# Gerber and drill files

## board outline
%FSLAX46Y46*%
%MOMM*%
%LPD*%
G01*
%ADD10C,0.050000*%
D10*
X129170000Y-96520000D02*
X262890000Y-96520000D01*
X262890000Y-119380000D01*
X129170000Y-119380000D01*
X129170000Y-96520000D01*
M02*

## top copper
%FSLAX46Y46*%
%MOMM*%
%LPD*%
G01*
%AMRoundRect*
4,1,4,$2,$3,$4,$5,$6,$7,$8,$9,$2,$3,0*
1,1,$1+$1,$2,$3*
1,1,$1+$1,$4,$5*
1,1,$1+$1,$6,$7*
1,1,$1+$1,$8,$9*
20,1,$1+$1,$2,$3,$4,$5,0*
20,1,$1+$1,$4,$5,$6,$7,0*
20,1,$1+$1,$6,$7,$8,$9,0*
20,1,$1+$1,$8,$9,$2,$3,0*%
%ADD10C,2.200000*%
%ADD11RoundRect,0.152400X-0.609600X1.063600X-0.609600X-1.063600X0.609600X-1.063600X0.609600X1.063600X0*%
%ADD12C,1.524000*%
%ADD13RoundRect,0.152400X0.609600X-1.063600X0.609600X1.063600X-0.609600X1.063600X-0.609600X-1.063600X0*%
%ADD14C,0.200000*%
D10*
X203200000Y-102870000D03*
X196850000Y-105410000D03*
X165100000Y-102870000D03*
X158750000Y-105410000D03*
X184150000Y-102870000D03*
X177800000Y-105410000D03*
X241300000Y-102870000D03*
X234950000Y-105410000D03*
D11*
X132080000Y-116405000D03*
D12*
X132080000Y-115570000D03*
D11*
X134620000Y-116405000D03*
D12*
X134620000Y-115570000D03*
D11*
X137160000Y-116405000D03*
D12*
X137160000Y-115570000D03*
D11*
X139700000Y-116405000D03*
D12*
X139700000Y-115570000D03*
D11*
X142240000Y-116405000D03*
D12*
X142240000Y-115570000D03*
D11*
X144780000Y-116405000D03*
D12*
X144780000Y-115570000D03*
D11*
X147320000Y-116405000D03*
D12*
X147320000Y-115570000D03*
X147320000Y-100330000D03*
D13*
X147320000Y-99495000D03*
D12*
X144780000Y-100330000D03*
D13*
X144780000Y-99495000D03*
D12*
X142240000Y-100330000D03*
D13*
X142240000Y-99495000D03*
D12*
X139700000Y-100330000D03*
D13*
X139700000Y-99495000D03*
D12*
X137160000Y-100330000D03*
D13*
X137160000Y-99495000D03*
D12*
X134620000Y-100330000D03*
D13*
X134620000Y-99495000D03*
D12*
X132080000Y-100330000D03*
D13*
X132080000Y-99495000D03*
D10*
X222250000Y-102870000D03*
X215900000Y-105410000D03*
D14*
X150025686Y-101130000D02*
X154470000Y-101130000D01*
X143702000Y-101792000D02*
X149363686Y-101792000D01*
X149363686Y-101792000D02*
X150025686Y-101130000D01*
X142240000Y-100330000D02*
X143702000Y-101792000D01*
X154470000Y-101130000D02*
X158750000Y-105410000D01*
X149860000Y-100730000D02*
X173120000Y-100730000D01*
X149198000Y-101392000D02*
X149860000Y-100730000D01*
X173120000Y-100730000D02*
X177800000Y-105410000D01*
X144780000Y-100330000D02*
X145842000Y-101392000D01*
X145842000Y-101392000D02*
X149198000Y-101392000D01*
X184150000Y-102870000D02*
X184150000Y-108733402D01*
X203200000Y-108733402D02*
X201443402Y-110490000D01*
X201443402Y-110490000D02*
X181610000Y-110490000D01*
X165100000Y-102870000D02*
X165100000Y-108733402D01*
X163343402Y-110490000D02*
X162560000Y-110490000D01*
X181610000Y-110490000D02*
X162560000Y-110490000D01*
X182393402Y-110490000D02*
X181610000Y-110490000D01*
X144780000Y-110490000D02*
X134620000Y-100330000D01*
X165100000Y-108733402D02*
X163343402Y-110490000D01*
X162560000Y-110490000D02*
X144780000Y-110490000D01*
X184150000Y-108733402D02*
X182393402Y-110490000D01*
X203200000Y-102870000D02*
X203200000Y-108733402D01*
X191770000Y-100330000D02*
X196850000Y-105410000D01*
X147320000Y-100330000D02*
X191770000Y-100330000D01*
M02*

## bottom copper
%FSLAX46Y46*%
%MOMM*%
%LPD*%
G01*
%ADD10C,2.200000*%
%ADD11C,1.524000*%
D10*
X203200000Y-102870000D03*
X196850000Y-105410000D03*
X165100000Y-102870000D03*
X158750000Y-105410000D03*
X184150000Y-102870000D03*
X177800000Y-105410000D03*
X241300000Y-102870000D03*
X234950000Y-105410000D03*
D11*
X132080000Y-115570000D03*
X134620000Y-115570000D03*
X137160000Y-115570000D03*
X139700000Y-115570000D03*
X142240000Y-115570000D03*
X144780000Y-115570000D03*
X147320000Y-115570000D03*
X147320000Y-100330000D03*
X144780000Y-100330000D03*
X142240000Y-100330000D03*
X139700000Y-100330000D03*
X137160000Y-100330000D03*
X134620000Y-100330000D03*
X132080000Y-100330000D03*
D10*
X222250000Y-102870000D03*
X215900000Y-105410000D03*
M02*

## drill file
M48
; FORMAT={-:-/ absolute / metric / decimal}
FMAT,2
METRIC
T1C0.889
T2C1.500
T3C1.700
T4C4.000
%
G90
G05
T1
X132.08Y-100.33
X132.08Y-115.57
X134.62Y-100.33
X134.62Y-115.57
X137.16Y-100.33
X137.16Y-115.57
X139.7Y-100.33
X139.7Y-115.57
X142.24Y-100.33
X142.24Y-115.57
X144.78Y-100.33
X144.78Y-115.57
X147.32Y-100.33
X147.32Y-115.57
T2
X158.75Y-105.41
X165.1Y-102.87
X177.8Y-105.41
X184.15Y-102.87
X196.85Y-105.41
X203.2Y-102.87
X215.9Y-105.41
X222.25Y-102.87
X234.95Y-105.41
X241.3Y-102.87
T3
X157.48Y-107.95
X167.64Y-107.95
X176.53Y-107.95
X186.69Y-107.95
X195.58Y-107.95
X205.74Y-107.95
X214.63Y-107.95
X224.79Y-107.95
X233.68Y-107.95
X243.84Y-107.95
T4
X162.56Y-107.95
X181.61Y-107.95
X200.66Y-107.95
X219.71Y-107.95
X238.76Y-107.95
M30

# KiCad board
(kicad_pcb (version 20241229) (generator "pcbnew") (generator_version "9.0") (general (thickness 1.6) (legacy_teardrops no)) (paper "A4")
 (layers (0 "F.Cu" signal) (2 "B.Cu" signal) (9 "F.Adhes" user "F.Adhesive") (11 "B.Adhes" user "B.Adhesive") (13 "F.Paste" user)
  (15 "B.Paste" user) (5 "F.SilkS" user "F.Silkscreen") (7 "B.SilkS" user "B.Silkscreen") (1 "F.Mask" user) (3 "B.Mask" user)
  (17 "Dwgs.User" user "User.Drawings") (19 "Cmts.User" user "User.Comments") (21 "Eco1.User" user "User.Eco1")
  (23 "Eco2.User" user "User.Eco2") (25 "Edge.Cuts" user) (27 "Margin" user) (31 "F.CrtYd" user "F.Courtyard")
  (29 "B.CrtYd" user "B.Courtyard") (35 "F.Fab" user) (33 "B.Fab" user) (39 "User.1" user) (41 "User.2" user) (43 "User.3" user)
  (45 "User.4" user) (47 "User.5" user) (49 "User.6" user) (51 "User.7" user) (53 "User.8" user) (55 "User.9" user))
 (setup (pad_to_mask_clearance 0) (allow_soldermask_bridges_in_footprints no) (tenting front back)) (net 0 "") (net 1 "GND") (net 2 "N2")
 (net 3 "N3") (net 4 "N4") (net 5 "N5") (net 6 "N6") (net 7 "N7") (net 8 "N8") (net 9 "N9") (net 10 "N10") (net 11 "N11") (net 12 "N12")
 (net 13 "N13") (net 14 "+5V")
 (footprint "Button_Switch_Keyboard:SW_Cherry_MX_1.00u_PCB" (layer "F.Cu") (at 203.2 102.87)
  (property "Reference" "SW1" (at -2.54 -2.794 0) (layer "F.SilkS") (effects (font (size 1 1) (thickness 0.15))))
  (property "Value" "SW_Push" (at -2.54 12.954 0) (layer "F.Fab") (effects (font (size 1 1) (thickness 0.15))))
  (pad "" np_thru_hole circle (at -7.62 5.08) (size 1.7 1.7) (drill 1.7) (layers "*.Cu" "*.Mask"))
  (pad "" np_thru_hole circle (at -2.54 5.08) (size 4 4) (drill 4) (layers "*.Cu" "*.Mask"))
  (pad "" np_thru_hole circle (at 2.54 5.08) (size 1.7 1.7) (drill 1.7) (layers "*.Cu" "*.Mask"))
  (pad "1" thru_hole circle (at 0 0) (size 2.2 2.2) (drill 1.5) (layers "*.Cu" "*.Mask") (remove_unused_layers no) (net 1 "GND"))
  (pad "2" thru_hole circle (at -6.35 2.54) (size 2.2 2.2) (drill 1.5) (layers "*.Cu" "*.Mask") (remove_unused_layers no) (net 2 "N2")))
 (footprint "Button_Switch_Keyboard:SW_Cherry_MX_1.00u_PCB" (layer "F.Cu") (at 165.1 102.87)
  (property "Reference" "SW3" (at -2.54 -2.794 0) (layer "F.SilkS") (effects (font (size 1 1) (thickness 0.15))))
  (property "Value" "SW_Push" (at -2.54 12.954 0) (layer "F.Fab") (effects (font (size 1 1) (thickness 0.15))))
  (pad "" np_thru_hole circle (at -7.62 5.08) (size 1.7 1.7) (drill 1.7) (layers "*.Cu" "*.Mask"))
  (pad "" np_thru_hole circle (at -2.54 5.08) (size 4 4) (drill 4) (layers "*.Cu" "*.Mask"))
  (pad "" np_thru_hole circle (at 2.54 5.08) (size 1.7 1.7) (drill 1.7) (layers "*.Cu" "*.Mask"))
  (pad "1" thru_hole circle (at 0 0) (size 2.2 2.2) (drill 1.5) (layers "*.Cu" "*.Mask") (remove_unused_layers no) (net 1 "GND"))
  (pad "2" thru_hole circle (at -6.35 2.54) (size 2.2 2.2) (drill 1.5) (layers "*.Cu" "*.Mask") (remove_unused_layers no) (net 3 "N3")))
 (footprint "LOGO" (layer "F.Cu") (at 253.109093 100.484313)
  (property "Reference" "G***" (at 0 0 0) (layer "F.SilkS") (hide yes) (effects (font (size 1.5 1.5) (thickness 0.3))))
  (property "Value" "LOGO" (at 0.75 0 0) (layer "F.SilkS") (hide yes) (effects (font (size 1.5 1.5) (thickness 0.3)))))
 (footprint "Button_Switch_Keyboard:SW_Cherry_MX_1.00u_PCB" (layer "F.Cu") (at 184.15 102.87)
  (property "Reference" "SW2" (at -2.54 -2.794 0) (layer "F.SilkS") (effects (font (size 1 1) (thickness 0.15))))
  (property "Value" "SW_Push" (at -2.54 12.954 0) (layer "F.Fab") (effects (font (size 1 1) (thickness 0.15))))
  (pad "" np_thru_hole circle (at -7.62 5.08) (size 1.7 1.7) (drill 1.7) (layers "*.Cu" "*.Mask"))
  (pad "" np_thru_hole circle (at -2.54 5.08) (size 4 4) (drill 4) (layers "*.Cu" "*.Mask"))
  (pad "" np_thru_hole circle (at 2.54 5.08) (size 1.7 1.7) (drill 1.7) (layers "*.Cu" "*.Mask"))
  (pad "1" thru_hole circle (at 0 0) (size 2.2 2.2) (drill 1.5) (layers "*.Cu" "*.Mask") (remove_unused_layers no) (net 1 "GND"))
  (pad "2" thru_hole circle (at -6.35 2.54) (size 2.2 2.2) (drill 1.5) (layers "*.Cu" "*.Mask") (remove_unused_layers no) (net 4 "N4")))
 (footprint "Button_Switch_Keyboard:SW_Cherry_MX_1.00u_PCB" (layer "F.Cu") (at 241.3 102.87)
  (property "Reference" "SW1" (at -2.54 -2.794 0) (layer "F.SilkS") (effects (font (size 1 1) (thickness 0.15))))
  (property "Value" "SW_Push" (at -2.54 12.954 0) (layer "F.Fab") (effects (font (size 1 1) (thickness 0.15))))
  (pad "" np_thru_hole circle (at -7.62 5.08) (size 1.7 1.7) (drill 1.7) (layers "*.Cu" "*.Mask"))
  (pad "" np_thru_hole circle (at -2.54 5.08) (size 4 4) (drill 4) (layers "*.Cu" "*.Mask"))
  (pad "" np_thru_hole circle (at 2.54 5.08) (size 1.7 1.7) (drill 1.7) (layers "*.Cu" "*.Mask"))
  (pad "1" thru_hole circle (at 0 0) (size 2.2 2.2) (drill 1.5) (layers "*.Cu" "*.Mask") (remove_unused_layers no))
  (pad "2" thru_hole circle (at -6.35 2.54) (size 2.2 2.2) (drill 1.5) (layers "*.Cu" "*.Mask") (remove_unused_layers no)))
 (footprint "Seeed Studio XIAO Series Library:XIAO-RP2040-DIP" (layer "F.Cu") (at 139.7 107.95 90)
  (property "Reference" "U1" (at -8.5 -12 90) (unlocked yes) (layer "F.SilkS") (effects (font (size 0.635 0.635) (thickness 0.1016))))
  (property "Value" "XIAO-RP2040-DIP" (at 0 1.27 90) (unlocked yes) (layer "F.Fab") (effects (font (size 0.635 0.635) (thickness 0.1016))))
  (pad "1" smd roundrect (at -8.455 -7.62 270) (size 2.432 1.524) (layers "F.Cu" "F.Mask") (roundrect_rratio 0.1) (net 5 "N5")
   (thermal_bridge_angle 45))
  (pad "1" thru_hole circle (at -7.62 -7.62 270) (size 1.524 1.524) (drill 0.889) (layers "*.Cu" "*.Mask") (remove_unused_layers no)
   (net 5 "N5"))
  (pad "2" smd roundrect (at -8.455 -5.08 270) (size 2.432 1.524) (layers "F.Cu" "F.Mask") (roundrect_rratio 0.1) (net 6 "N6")
   (thermal_bridge_angle 45))
  (pad "2" thru_hole circle (at -7.62 -5.08 270) (size 1.524 1.524) (drill 0.889) (layers "*.Cu" "*.Mask") (remove_unused_layers no)
   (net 6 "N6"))
  (pad "3" smd roundrect (at -8.455 -2.54 270) (size 2.432 1.524) (layers "F.Cu" "F.Mask") (roundrect_rratio 0.1) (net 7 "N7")
   (thermal_bridge_angle 45))
  (pad "3" thru_hole circle (at -7.62 -2.54 270) (size 1.524 1.524) (drill 0.889) (layers "*.Cu" "*.Mask") (remove_unused_layers no)
   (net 7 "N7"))
  (pad "4" smd roundrect (at -8.455 0 270) (size 2.432 1.524) (layers "F.Cu" "F.Mask") (roundrect_rratio 0.1) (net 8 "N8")
   (thermal_bridge_angle 45))
  (pad "4" thru_hole circle (at -7.62 0 270) (size 1.524 1.524) (drill 0.889) (layers "*.Cu" "*.Mask") (remove_unused_layers no)
   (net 8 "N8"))
  (pad "5" smd roundrect (at -8.455 2.54 270) (size 2.432 1.524) (layers "F.Cu" "F.Mask") (roundrect_rratio 0.1) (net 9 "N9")
   (thermal_bridge_angle 45))
  (pad "5" thru_hole circle (at -7.62 2.54 270) (size 1.524 1.524) (drill 0.889) (layers "*.Cu" "*.Mask") (remove_unused_layers no)
   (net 9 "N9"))
  (pad "6" smd roundrect (at -8.455 5.08 270) (size 2.432 1.524) (layers "F.Cu" "F.Mask") (roundrect_rratio 0.1) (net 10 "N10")
   (thermal_bridge_angle 45))
  (pad "6" thru_hole circle (at -7.62 5.08 270) (size 1.524 1.524) (drill 0.889) (layers "*.Cu" "*.Mask") (remove_unused_layers no)
   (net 10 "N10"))
  (pad "7" smd roundrect (at -8.455 7.62 270) (size 2.432 1.524) (layers "F.Cu" "F.Mask") (roundrect_rratio 0.1) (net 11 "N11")
   (thermal_bridge_angle 45))
  (pad "7" thru_hole circle (at -7.62 7.62 270) (size 1.524 1.524) (drill 0.889) (layers "*.Cu" "*.Mask") (remove_unused_layers no)
   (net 11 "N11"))
  (pad "8" thru_hole circle (at 7.62 7.62 90) (size 1.524 1.524) (drill 0.889) (layers "*.Cu" "*.Mask") (remove_unused_layers no)
   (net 2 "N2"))
  (pad "8" smd roundrect (at 8.455 7.62 90) (size 2.432 1.524) (layers "F.Cu" "F.Mask") (roundrect_rratio 0.1) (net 2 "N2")
   (thermal_bridge_angle 45))
  (pad "9" thru_hole circle (at 7.62 5.08 90) (size 1.524 1.524) (drill 0.889) (layers "*.Cu" "*.Mask") (remove_unused_layers no)
   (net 4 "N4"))
  (pad "9" smd roundrect (at 8.455 5.08 90) (size 2.432 1.524) (layers "F.Cu" "F.Mask") (roundrect_rratio 0.1) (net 4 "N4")
   (thermal_bridge_angle 45))
  (pad "10" thru_hole circle (at 7.62 2.54 90) (size 1.524 1.524) (drill 0.889) (layers "*.Cu" "*.Mask") (remove_unused_layers no)
   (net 3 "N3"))
  (pad "10" smd roundrect (at 8.455 2.54 90) (size 2.432 1.524) (layers "F.Cu" "F.Mask") (roundrect_rratio 0.1) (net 3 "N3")
   (thermal_bridge_angle 45))
  (pad "11" thru_hole circle (at 7.62 0 90) (size 1.524 1.524) (drill 0.889) (layers "*.Cu" "*.Mask") (remove_unused_layers no)
   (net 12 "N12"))
  (pad "11" smd roundrect (at 8.455 0 90) (size 2.432 1.524) (layers "F.Cu" "F.Mask") (roundrect_rratio 0.1) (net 12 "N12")
   (thermal_bridge_angle 45))
  (pad "12" thru_hole circle (at 7.62 -2.54 90) (size 1.524 1.524) (drill 0.889) (layers "*.Cu" "*.Mask") (remove_unused_layers no)
   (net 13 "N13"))
  (pad "12" smd roundrect (at 8.455 -2.54 90) (size 2.432 1.524) (layers "F.Cu" "F.Mask") (roundrect_rratio 0.1) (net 13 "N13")
   (thermal_bridge_angle 45))
  (pad "13" thru_hole circle (at 7.62 -5.08 90) (size 1.524 1.524) (drill 0.889) (layers "*.Cu" "*.Mask") (remove_unused_layers no)
   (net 1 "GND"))
  (pad "13" smd roundrect (at 8.455 -5.08 90) (size 2.432 1.524) (layers "F.Cu" "F.Mask") (roundrect_rratio 0.1) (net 1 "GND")
   (thermal_bridge_angle 45))
  (pad "14" thru_hole circle (at 7.62 -7.62 90) (size 1.524 1.524) (drill 0.889) (layers "*.Cu" "*.Mask") (remove_unused_layers no)
   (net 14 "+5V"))
  (pad "14" smd roundrect (at 8.455 -7.62 90) (size 2.432 1.524) (layers "F.Cu" "F.Mask") (roundrect_rratio 0.1) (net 14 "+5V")
   (thermal_bridge_angle 45)))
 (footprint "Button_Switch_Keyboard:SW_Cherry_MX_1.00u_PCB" (layer "F.Cu") (at 222.25 102.87)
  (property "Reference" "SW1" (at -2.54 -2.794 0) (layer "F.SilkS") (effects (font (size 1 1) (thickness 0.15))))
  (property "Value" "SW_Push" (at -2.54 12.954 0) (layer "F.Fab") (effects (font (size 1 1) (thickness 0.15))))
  (pad "" np_thru_hole circle (at -7.62 5.08) (size 1.7 1.7) (drill 1.7) (layers "*.Cu" "*.Mask"))
  (pad "" np_thru_hole circle (at -2.54 5.08) (size 4 4) (drill 4) (layers "*.Cu" "*.Mask"))
  (pad "" np_thru_hole circle (at 2.54 5.08) (size 1.7 1.7) (drill 1.7) (layers "*.Cu" "*.Mask"))
  (pad "1" thru_hole circle (at 0 0) (size 2.2 2.2) (drill 1.5) (layers "*.Cu" "*.Mask") (remove_unused_layers no))
  (pad "2" thru_hole circle (at -6.35 2.54) (size 2.2 2.2) (drill 1.5) (layers "*.Cu" "*.Mask") (remove_unused_layers no)))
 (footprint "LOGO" (layer "F.Cu") (at 255.718534 111.483751)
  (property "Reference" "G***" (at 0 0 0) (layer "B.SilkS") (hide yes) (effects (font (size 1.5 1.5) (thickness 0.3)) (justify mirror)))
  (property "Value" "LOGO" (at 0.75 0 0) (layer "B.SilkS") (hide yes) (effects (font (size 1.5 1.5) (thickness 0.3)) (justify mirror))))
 (gr_rect (start 129.17 96.52) (end 262.89 119.38) (stroke (width 0.05) (type default)) (fill no) (layer "Edge.Cuts"))
 (segment (start 150.025686 101.13) (end 154.47 101.13) (width 0.2) (layer "F.Cu") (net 3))
 (segment (start 143.702 101.792) (end 149.363686 101.792) (width 0.2) (layer "F.Cu") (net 3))
 (segment (start 149.363686 101.792) (end 150.025686 101.13) (width 0.2) (layer "F.Cu") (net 3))
 (segment (start 142.24 100.33) (end 143.702 101.792) (width 0.2) (layer "F.Cu") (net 3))
 (segment (start 154.47 101.13) (end 158.75 105.41) (width 0.2) (layer "F.Cu") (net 3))
 (segment (start 149.86 100.73) (end 173.12 100.73) (width 0.2) (layer "F.Cu") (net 4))
 (segment (start 149.198 101.392) (end 149.86 100.73) (width 0.2) (layer "F.Cu") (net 4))
 (segment (start 173.12 100.73) (end 177.8 105.41) (width 0.2) (layer "F.Cu") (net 4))
 (segment (start 144.78 100.33) (end 145.842 101.392) (width 0.2) (layer "F.Cu") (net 4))
 (segment (start 145.842 101.392) (end 149.198 101.392) (width 0.2) (layer "F.Cu") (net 4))
 (segment (start 184.15 102.87) (end 184.15 108.733402) (width 0.2) (layer "F.Cu") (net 1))
 (segment (start 203.2 108.733402) (end 201.443402 110.49) (width 0.2) (layer "F.Cu") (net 1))
 (segment (start 201.443402 110.49) (end 181.61 110.49) (width 0.2) (layer "F.Cu") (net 1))
 (segment (start 165.1 102.87) (end 165.1 108.733402) (width 0.2) (layer "F.Cu") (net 1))
 (segment (start 163.343402 110.49) (end 162.56 110.49) (width 0.2) (layer "F.Cu") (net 1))
 (segment (start 181.61 110.49) (end 162.56 110.49) (width 0.2) (layer "F.Cu") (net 1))
 (segment (start 182.393402 110.49) (end 181.61 110.49) (width 0.2) (layer "F.Cu") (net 1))
 (segment (start 144.78 110.49) (end 134.62 100.33) (width 0.2) (layer "F.Cu") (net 1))
 (segment (start 165.1 108.733402) (end 163.343402 110.49) (width 0.2) (layer "F.Cu") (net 1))
 (segment (start 162.56 110.49) (end 144.78 110.49) (width 0.2) (layer "F.Cu") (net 1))
 (segment (start 184.15 108.733402) (end 182.393402 110.49) (width 0.2) (layer "F.Cu") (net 1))
 (segment (start 203.2 102.87) (end 203.2 108.733402) (width 0.2) (layer "F.Cu") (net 1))
 (segment (start 191.77 100.33) (end 196.85 105.41) (width 0.2) (layer "F.Cu") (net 2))
 (segment (start 147.32 100.33) (end 191.77 100.33) (width 0.2) (layer "F.Cu") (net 2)))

